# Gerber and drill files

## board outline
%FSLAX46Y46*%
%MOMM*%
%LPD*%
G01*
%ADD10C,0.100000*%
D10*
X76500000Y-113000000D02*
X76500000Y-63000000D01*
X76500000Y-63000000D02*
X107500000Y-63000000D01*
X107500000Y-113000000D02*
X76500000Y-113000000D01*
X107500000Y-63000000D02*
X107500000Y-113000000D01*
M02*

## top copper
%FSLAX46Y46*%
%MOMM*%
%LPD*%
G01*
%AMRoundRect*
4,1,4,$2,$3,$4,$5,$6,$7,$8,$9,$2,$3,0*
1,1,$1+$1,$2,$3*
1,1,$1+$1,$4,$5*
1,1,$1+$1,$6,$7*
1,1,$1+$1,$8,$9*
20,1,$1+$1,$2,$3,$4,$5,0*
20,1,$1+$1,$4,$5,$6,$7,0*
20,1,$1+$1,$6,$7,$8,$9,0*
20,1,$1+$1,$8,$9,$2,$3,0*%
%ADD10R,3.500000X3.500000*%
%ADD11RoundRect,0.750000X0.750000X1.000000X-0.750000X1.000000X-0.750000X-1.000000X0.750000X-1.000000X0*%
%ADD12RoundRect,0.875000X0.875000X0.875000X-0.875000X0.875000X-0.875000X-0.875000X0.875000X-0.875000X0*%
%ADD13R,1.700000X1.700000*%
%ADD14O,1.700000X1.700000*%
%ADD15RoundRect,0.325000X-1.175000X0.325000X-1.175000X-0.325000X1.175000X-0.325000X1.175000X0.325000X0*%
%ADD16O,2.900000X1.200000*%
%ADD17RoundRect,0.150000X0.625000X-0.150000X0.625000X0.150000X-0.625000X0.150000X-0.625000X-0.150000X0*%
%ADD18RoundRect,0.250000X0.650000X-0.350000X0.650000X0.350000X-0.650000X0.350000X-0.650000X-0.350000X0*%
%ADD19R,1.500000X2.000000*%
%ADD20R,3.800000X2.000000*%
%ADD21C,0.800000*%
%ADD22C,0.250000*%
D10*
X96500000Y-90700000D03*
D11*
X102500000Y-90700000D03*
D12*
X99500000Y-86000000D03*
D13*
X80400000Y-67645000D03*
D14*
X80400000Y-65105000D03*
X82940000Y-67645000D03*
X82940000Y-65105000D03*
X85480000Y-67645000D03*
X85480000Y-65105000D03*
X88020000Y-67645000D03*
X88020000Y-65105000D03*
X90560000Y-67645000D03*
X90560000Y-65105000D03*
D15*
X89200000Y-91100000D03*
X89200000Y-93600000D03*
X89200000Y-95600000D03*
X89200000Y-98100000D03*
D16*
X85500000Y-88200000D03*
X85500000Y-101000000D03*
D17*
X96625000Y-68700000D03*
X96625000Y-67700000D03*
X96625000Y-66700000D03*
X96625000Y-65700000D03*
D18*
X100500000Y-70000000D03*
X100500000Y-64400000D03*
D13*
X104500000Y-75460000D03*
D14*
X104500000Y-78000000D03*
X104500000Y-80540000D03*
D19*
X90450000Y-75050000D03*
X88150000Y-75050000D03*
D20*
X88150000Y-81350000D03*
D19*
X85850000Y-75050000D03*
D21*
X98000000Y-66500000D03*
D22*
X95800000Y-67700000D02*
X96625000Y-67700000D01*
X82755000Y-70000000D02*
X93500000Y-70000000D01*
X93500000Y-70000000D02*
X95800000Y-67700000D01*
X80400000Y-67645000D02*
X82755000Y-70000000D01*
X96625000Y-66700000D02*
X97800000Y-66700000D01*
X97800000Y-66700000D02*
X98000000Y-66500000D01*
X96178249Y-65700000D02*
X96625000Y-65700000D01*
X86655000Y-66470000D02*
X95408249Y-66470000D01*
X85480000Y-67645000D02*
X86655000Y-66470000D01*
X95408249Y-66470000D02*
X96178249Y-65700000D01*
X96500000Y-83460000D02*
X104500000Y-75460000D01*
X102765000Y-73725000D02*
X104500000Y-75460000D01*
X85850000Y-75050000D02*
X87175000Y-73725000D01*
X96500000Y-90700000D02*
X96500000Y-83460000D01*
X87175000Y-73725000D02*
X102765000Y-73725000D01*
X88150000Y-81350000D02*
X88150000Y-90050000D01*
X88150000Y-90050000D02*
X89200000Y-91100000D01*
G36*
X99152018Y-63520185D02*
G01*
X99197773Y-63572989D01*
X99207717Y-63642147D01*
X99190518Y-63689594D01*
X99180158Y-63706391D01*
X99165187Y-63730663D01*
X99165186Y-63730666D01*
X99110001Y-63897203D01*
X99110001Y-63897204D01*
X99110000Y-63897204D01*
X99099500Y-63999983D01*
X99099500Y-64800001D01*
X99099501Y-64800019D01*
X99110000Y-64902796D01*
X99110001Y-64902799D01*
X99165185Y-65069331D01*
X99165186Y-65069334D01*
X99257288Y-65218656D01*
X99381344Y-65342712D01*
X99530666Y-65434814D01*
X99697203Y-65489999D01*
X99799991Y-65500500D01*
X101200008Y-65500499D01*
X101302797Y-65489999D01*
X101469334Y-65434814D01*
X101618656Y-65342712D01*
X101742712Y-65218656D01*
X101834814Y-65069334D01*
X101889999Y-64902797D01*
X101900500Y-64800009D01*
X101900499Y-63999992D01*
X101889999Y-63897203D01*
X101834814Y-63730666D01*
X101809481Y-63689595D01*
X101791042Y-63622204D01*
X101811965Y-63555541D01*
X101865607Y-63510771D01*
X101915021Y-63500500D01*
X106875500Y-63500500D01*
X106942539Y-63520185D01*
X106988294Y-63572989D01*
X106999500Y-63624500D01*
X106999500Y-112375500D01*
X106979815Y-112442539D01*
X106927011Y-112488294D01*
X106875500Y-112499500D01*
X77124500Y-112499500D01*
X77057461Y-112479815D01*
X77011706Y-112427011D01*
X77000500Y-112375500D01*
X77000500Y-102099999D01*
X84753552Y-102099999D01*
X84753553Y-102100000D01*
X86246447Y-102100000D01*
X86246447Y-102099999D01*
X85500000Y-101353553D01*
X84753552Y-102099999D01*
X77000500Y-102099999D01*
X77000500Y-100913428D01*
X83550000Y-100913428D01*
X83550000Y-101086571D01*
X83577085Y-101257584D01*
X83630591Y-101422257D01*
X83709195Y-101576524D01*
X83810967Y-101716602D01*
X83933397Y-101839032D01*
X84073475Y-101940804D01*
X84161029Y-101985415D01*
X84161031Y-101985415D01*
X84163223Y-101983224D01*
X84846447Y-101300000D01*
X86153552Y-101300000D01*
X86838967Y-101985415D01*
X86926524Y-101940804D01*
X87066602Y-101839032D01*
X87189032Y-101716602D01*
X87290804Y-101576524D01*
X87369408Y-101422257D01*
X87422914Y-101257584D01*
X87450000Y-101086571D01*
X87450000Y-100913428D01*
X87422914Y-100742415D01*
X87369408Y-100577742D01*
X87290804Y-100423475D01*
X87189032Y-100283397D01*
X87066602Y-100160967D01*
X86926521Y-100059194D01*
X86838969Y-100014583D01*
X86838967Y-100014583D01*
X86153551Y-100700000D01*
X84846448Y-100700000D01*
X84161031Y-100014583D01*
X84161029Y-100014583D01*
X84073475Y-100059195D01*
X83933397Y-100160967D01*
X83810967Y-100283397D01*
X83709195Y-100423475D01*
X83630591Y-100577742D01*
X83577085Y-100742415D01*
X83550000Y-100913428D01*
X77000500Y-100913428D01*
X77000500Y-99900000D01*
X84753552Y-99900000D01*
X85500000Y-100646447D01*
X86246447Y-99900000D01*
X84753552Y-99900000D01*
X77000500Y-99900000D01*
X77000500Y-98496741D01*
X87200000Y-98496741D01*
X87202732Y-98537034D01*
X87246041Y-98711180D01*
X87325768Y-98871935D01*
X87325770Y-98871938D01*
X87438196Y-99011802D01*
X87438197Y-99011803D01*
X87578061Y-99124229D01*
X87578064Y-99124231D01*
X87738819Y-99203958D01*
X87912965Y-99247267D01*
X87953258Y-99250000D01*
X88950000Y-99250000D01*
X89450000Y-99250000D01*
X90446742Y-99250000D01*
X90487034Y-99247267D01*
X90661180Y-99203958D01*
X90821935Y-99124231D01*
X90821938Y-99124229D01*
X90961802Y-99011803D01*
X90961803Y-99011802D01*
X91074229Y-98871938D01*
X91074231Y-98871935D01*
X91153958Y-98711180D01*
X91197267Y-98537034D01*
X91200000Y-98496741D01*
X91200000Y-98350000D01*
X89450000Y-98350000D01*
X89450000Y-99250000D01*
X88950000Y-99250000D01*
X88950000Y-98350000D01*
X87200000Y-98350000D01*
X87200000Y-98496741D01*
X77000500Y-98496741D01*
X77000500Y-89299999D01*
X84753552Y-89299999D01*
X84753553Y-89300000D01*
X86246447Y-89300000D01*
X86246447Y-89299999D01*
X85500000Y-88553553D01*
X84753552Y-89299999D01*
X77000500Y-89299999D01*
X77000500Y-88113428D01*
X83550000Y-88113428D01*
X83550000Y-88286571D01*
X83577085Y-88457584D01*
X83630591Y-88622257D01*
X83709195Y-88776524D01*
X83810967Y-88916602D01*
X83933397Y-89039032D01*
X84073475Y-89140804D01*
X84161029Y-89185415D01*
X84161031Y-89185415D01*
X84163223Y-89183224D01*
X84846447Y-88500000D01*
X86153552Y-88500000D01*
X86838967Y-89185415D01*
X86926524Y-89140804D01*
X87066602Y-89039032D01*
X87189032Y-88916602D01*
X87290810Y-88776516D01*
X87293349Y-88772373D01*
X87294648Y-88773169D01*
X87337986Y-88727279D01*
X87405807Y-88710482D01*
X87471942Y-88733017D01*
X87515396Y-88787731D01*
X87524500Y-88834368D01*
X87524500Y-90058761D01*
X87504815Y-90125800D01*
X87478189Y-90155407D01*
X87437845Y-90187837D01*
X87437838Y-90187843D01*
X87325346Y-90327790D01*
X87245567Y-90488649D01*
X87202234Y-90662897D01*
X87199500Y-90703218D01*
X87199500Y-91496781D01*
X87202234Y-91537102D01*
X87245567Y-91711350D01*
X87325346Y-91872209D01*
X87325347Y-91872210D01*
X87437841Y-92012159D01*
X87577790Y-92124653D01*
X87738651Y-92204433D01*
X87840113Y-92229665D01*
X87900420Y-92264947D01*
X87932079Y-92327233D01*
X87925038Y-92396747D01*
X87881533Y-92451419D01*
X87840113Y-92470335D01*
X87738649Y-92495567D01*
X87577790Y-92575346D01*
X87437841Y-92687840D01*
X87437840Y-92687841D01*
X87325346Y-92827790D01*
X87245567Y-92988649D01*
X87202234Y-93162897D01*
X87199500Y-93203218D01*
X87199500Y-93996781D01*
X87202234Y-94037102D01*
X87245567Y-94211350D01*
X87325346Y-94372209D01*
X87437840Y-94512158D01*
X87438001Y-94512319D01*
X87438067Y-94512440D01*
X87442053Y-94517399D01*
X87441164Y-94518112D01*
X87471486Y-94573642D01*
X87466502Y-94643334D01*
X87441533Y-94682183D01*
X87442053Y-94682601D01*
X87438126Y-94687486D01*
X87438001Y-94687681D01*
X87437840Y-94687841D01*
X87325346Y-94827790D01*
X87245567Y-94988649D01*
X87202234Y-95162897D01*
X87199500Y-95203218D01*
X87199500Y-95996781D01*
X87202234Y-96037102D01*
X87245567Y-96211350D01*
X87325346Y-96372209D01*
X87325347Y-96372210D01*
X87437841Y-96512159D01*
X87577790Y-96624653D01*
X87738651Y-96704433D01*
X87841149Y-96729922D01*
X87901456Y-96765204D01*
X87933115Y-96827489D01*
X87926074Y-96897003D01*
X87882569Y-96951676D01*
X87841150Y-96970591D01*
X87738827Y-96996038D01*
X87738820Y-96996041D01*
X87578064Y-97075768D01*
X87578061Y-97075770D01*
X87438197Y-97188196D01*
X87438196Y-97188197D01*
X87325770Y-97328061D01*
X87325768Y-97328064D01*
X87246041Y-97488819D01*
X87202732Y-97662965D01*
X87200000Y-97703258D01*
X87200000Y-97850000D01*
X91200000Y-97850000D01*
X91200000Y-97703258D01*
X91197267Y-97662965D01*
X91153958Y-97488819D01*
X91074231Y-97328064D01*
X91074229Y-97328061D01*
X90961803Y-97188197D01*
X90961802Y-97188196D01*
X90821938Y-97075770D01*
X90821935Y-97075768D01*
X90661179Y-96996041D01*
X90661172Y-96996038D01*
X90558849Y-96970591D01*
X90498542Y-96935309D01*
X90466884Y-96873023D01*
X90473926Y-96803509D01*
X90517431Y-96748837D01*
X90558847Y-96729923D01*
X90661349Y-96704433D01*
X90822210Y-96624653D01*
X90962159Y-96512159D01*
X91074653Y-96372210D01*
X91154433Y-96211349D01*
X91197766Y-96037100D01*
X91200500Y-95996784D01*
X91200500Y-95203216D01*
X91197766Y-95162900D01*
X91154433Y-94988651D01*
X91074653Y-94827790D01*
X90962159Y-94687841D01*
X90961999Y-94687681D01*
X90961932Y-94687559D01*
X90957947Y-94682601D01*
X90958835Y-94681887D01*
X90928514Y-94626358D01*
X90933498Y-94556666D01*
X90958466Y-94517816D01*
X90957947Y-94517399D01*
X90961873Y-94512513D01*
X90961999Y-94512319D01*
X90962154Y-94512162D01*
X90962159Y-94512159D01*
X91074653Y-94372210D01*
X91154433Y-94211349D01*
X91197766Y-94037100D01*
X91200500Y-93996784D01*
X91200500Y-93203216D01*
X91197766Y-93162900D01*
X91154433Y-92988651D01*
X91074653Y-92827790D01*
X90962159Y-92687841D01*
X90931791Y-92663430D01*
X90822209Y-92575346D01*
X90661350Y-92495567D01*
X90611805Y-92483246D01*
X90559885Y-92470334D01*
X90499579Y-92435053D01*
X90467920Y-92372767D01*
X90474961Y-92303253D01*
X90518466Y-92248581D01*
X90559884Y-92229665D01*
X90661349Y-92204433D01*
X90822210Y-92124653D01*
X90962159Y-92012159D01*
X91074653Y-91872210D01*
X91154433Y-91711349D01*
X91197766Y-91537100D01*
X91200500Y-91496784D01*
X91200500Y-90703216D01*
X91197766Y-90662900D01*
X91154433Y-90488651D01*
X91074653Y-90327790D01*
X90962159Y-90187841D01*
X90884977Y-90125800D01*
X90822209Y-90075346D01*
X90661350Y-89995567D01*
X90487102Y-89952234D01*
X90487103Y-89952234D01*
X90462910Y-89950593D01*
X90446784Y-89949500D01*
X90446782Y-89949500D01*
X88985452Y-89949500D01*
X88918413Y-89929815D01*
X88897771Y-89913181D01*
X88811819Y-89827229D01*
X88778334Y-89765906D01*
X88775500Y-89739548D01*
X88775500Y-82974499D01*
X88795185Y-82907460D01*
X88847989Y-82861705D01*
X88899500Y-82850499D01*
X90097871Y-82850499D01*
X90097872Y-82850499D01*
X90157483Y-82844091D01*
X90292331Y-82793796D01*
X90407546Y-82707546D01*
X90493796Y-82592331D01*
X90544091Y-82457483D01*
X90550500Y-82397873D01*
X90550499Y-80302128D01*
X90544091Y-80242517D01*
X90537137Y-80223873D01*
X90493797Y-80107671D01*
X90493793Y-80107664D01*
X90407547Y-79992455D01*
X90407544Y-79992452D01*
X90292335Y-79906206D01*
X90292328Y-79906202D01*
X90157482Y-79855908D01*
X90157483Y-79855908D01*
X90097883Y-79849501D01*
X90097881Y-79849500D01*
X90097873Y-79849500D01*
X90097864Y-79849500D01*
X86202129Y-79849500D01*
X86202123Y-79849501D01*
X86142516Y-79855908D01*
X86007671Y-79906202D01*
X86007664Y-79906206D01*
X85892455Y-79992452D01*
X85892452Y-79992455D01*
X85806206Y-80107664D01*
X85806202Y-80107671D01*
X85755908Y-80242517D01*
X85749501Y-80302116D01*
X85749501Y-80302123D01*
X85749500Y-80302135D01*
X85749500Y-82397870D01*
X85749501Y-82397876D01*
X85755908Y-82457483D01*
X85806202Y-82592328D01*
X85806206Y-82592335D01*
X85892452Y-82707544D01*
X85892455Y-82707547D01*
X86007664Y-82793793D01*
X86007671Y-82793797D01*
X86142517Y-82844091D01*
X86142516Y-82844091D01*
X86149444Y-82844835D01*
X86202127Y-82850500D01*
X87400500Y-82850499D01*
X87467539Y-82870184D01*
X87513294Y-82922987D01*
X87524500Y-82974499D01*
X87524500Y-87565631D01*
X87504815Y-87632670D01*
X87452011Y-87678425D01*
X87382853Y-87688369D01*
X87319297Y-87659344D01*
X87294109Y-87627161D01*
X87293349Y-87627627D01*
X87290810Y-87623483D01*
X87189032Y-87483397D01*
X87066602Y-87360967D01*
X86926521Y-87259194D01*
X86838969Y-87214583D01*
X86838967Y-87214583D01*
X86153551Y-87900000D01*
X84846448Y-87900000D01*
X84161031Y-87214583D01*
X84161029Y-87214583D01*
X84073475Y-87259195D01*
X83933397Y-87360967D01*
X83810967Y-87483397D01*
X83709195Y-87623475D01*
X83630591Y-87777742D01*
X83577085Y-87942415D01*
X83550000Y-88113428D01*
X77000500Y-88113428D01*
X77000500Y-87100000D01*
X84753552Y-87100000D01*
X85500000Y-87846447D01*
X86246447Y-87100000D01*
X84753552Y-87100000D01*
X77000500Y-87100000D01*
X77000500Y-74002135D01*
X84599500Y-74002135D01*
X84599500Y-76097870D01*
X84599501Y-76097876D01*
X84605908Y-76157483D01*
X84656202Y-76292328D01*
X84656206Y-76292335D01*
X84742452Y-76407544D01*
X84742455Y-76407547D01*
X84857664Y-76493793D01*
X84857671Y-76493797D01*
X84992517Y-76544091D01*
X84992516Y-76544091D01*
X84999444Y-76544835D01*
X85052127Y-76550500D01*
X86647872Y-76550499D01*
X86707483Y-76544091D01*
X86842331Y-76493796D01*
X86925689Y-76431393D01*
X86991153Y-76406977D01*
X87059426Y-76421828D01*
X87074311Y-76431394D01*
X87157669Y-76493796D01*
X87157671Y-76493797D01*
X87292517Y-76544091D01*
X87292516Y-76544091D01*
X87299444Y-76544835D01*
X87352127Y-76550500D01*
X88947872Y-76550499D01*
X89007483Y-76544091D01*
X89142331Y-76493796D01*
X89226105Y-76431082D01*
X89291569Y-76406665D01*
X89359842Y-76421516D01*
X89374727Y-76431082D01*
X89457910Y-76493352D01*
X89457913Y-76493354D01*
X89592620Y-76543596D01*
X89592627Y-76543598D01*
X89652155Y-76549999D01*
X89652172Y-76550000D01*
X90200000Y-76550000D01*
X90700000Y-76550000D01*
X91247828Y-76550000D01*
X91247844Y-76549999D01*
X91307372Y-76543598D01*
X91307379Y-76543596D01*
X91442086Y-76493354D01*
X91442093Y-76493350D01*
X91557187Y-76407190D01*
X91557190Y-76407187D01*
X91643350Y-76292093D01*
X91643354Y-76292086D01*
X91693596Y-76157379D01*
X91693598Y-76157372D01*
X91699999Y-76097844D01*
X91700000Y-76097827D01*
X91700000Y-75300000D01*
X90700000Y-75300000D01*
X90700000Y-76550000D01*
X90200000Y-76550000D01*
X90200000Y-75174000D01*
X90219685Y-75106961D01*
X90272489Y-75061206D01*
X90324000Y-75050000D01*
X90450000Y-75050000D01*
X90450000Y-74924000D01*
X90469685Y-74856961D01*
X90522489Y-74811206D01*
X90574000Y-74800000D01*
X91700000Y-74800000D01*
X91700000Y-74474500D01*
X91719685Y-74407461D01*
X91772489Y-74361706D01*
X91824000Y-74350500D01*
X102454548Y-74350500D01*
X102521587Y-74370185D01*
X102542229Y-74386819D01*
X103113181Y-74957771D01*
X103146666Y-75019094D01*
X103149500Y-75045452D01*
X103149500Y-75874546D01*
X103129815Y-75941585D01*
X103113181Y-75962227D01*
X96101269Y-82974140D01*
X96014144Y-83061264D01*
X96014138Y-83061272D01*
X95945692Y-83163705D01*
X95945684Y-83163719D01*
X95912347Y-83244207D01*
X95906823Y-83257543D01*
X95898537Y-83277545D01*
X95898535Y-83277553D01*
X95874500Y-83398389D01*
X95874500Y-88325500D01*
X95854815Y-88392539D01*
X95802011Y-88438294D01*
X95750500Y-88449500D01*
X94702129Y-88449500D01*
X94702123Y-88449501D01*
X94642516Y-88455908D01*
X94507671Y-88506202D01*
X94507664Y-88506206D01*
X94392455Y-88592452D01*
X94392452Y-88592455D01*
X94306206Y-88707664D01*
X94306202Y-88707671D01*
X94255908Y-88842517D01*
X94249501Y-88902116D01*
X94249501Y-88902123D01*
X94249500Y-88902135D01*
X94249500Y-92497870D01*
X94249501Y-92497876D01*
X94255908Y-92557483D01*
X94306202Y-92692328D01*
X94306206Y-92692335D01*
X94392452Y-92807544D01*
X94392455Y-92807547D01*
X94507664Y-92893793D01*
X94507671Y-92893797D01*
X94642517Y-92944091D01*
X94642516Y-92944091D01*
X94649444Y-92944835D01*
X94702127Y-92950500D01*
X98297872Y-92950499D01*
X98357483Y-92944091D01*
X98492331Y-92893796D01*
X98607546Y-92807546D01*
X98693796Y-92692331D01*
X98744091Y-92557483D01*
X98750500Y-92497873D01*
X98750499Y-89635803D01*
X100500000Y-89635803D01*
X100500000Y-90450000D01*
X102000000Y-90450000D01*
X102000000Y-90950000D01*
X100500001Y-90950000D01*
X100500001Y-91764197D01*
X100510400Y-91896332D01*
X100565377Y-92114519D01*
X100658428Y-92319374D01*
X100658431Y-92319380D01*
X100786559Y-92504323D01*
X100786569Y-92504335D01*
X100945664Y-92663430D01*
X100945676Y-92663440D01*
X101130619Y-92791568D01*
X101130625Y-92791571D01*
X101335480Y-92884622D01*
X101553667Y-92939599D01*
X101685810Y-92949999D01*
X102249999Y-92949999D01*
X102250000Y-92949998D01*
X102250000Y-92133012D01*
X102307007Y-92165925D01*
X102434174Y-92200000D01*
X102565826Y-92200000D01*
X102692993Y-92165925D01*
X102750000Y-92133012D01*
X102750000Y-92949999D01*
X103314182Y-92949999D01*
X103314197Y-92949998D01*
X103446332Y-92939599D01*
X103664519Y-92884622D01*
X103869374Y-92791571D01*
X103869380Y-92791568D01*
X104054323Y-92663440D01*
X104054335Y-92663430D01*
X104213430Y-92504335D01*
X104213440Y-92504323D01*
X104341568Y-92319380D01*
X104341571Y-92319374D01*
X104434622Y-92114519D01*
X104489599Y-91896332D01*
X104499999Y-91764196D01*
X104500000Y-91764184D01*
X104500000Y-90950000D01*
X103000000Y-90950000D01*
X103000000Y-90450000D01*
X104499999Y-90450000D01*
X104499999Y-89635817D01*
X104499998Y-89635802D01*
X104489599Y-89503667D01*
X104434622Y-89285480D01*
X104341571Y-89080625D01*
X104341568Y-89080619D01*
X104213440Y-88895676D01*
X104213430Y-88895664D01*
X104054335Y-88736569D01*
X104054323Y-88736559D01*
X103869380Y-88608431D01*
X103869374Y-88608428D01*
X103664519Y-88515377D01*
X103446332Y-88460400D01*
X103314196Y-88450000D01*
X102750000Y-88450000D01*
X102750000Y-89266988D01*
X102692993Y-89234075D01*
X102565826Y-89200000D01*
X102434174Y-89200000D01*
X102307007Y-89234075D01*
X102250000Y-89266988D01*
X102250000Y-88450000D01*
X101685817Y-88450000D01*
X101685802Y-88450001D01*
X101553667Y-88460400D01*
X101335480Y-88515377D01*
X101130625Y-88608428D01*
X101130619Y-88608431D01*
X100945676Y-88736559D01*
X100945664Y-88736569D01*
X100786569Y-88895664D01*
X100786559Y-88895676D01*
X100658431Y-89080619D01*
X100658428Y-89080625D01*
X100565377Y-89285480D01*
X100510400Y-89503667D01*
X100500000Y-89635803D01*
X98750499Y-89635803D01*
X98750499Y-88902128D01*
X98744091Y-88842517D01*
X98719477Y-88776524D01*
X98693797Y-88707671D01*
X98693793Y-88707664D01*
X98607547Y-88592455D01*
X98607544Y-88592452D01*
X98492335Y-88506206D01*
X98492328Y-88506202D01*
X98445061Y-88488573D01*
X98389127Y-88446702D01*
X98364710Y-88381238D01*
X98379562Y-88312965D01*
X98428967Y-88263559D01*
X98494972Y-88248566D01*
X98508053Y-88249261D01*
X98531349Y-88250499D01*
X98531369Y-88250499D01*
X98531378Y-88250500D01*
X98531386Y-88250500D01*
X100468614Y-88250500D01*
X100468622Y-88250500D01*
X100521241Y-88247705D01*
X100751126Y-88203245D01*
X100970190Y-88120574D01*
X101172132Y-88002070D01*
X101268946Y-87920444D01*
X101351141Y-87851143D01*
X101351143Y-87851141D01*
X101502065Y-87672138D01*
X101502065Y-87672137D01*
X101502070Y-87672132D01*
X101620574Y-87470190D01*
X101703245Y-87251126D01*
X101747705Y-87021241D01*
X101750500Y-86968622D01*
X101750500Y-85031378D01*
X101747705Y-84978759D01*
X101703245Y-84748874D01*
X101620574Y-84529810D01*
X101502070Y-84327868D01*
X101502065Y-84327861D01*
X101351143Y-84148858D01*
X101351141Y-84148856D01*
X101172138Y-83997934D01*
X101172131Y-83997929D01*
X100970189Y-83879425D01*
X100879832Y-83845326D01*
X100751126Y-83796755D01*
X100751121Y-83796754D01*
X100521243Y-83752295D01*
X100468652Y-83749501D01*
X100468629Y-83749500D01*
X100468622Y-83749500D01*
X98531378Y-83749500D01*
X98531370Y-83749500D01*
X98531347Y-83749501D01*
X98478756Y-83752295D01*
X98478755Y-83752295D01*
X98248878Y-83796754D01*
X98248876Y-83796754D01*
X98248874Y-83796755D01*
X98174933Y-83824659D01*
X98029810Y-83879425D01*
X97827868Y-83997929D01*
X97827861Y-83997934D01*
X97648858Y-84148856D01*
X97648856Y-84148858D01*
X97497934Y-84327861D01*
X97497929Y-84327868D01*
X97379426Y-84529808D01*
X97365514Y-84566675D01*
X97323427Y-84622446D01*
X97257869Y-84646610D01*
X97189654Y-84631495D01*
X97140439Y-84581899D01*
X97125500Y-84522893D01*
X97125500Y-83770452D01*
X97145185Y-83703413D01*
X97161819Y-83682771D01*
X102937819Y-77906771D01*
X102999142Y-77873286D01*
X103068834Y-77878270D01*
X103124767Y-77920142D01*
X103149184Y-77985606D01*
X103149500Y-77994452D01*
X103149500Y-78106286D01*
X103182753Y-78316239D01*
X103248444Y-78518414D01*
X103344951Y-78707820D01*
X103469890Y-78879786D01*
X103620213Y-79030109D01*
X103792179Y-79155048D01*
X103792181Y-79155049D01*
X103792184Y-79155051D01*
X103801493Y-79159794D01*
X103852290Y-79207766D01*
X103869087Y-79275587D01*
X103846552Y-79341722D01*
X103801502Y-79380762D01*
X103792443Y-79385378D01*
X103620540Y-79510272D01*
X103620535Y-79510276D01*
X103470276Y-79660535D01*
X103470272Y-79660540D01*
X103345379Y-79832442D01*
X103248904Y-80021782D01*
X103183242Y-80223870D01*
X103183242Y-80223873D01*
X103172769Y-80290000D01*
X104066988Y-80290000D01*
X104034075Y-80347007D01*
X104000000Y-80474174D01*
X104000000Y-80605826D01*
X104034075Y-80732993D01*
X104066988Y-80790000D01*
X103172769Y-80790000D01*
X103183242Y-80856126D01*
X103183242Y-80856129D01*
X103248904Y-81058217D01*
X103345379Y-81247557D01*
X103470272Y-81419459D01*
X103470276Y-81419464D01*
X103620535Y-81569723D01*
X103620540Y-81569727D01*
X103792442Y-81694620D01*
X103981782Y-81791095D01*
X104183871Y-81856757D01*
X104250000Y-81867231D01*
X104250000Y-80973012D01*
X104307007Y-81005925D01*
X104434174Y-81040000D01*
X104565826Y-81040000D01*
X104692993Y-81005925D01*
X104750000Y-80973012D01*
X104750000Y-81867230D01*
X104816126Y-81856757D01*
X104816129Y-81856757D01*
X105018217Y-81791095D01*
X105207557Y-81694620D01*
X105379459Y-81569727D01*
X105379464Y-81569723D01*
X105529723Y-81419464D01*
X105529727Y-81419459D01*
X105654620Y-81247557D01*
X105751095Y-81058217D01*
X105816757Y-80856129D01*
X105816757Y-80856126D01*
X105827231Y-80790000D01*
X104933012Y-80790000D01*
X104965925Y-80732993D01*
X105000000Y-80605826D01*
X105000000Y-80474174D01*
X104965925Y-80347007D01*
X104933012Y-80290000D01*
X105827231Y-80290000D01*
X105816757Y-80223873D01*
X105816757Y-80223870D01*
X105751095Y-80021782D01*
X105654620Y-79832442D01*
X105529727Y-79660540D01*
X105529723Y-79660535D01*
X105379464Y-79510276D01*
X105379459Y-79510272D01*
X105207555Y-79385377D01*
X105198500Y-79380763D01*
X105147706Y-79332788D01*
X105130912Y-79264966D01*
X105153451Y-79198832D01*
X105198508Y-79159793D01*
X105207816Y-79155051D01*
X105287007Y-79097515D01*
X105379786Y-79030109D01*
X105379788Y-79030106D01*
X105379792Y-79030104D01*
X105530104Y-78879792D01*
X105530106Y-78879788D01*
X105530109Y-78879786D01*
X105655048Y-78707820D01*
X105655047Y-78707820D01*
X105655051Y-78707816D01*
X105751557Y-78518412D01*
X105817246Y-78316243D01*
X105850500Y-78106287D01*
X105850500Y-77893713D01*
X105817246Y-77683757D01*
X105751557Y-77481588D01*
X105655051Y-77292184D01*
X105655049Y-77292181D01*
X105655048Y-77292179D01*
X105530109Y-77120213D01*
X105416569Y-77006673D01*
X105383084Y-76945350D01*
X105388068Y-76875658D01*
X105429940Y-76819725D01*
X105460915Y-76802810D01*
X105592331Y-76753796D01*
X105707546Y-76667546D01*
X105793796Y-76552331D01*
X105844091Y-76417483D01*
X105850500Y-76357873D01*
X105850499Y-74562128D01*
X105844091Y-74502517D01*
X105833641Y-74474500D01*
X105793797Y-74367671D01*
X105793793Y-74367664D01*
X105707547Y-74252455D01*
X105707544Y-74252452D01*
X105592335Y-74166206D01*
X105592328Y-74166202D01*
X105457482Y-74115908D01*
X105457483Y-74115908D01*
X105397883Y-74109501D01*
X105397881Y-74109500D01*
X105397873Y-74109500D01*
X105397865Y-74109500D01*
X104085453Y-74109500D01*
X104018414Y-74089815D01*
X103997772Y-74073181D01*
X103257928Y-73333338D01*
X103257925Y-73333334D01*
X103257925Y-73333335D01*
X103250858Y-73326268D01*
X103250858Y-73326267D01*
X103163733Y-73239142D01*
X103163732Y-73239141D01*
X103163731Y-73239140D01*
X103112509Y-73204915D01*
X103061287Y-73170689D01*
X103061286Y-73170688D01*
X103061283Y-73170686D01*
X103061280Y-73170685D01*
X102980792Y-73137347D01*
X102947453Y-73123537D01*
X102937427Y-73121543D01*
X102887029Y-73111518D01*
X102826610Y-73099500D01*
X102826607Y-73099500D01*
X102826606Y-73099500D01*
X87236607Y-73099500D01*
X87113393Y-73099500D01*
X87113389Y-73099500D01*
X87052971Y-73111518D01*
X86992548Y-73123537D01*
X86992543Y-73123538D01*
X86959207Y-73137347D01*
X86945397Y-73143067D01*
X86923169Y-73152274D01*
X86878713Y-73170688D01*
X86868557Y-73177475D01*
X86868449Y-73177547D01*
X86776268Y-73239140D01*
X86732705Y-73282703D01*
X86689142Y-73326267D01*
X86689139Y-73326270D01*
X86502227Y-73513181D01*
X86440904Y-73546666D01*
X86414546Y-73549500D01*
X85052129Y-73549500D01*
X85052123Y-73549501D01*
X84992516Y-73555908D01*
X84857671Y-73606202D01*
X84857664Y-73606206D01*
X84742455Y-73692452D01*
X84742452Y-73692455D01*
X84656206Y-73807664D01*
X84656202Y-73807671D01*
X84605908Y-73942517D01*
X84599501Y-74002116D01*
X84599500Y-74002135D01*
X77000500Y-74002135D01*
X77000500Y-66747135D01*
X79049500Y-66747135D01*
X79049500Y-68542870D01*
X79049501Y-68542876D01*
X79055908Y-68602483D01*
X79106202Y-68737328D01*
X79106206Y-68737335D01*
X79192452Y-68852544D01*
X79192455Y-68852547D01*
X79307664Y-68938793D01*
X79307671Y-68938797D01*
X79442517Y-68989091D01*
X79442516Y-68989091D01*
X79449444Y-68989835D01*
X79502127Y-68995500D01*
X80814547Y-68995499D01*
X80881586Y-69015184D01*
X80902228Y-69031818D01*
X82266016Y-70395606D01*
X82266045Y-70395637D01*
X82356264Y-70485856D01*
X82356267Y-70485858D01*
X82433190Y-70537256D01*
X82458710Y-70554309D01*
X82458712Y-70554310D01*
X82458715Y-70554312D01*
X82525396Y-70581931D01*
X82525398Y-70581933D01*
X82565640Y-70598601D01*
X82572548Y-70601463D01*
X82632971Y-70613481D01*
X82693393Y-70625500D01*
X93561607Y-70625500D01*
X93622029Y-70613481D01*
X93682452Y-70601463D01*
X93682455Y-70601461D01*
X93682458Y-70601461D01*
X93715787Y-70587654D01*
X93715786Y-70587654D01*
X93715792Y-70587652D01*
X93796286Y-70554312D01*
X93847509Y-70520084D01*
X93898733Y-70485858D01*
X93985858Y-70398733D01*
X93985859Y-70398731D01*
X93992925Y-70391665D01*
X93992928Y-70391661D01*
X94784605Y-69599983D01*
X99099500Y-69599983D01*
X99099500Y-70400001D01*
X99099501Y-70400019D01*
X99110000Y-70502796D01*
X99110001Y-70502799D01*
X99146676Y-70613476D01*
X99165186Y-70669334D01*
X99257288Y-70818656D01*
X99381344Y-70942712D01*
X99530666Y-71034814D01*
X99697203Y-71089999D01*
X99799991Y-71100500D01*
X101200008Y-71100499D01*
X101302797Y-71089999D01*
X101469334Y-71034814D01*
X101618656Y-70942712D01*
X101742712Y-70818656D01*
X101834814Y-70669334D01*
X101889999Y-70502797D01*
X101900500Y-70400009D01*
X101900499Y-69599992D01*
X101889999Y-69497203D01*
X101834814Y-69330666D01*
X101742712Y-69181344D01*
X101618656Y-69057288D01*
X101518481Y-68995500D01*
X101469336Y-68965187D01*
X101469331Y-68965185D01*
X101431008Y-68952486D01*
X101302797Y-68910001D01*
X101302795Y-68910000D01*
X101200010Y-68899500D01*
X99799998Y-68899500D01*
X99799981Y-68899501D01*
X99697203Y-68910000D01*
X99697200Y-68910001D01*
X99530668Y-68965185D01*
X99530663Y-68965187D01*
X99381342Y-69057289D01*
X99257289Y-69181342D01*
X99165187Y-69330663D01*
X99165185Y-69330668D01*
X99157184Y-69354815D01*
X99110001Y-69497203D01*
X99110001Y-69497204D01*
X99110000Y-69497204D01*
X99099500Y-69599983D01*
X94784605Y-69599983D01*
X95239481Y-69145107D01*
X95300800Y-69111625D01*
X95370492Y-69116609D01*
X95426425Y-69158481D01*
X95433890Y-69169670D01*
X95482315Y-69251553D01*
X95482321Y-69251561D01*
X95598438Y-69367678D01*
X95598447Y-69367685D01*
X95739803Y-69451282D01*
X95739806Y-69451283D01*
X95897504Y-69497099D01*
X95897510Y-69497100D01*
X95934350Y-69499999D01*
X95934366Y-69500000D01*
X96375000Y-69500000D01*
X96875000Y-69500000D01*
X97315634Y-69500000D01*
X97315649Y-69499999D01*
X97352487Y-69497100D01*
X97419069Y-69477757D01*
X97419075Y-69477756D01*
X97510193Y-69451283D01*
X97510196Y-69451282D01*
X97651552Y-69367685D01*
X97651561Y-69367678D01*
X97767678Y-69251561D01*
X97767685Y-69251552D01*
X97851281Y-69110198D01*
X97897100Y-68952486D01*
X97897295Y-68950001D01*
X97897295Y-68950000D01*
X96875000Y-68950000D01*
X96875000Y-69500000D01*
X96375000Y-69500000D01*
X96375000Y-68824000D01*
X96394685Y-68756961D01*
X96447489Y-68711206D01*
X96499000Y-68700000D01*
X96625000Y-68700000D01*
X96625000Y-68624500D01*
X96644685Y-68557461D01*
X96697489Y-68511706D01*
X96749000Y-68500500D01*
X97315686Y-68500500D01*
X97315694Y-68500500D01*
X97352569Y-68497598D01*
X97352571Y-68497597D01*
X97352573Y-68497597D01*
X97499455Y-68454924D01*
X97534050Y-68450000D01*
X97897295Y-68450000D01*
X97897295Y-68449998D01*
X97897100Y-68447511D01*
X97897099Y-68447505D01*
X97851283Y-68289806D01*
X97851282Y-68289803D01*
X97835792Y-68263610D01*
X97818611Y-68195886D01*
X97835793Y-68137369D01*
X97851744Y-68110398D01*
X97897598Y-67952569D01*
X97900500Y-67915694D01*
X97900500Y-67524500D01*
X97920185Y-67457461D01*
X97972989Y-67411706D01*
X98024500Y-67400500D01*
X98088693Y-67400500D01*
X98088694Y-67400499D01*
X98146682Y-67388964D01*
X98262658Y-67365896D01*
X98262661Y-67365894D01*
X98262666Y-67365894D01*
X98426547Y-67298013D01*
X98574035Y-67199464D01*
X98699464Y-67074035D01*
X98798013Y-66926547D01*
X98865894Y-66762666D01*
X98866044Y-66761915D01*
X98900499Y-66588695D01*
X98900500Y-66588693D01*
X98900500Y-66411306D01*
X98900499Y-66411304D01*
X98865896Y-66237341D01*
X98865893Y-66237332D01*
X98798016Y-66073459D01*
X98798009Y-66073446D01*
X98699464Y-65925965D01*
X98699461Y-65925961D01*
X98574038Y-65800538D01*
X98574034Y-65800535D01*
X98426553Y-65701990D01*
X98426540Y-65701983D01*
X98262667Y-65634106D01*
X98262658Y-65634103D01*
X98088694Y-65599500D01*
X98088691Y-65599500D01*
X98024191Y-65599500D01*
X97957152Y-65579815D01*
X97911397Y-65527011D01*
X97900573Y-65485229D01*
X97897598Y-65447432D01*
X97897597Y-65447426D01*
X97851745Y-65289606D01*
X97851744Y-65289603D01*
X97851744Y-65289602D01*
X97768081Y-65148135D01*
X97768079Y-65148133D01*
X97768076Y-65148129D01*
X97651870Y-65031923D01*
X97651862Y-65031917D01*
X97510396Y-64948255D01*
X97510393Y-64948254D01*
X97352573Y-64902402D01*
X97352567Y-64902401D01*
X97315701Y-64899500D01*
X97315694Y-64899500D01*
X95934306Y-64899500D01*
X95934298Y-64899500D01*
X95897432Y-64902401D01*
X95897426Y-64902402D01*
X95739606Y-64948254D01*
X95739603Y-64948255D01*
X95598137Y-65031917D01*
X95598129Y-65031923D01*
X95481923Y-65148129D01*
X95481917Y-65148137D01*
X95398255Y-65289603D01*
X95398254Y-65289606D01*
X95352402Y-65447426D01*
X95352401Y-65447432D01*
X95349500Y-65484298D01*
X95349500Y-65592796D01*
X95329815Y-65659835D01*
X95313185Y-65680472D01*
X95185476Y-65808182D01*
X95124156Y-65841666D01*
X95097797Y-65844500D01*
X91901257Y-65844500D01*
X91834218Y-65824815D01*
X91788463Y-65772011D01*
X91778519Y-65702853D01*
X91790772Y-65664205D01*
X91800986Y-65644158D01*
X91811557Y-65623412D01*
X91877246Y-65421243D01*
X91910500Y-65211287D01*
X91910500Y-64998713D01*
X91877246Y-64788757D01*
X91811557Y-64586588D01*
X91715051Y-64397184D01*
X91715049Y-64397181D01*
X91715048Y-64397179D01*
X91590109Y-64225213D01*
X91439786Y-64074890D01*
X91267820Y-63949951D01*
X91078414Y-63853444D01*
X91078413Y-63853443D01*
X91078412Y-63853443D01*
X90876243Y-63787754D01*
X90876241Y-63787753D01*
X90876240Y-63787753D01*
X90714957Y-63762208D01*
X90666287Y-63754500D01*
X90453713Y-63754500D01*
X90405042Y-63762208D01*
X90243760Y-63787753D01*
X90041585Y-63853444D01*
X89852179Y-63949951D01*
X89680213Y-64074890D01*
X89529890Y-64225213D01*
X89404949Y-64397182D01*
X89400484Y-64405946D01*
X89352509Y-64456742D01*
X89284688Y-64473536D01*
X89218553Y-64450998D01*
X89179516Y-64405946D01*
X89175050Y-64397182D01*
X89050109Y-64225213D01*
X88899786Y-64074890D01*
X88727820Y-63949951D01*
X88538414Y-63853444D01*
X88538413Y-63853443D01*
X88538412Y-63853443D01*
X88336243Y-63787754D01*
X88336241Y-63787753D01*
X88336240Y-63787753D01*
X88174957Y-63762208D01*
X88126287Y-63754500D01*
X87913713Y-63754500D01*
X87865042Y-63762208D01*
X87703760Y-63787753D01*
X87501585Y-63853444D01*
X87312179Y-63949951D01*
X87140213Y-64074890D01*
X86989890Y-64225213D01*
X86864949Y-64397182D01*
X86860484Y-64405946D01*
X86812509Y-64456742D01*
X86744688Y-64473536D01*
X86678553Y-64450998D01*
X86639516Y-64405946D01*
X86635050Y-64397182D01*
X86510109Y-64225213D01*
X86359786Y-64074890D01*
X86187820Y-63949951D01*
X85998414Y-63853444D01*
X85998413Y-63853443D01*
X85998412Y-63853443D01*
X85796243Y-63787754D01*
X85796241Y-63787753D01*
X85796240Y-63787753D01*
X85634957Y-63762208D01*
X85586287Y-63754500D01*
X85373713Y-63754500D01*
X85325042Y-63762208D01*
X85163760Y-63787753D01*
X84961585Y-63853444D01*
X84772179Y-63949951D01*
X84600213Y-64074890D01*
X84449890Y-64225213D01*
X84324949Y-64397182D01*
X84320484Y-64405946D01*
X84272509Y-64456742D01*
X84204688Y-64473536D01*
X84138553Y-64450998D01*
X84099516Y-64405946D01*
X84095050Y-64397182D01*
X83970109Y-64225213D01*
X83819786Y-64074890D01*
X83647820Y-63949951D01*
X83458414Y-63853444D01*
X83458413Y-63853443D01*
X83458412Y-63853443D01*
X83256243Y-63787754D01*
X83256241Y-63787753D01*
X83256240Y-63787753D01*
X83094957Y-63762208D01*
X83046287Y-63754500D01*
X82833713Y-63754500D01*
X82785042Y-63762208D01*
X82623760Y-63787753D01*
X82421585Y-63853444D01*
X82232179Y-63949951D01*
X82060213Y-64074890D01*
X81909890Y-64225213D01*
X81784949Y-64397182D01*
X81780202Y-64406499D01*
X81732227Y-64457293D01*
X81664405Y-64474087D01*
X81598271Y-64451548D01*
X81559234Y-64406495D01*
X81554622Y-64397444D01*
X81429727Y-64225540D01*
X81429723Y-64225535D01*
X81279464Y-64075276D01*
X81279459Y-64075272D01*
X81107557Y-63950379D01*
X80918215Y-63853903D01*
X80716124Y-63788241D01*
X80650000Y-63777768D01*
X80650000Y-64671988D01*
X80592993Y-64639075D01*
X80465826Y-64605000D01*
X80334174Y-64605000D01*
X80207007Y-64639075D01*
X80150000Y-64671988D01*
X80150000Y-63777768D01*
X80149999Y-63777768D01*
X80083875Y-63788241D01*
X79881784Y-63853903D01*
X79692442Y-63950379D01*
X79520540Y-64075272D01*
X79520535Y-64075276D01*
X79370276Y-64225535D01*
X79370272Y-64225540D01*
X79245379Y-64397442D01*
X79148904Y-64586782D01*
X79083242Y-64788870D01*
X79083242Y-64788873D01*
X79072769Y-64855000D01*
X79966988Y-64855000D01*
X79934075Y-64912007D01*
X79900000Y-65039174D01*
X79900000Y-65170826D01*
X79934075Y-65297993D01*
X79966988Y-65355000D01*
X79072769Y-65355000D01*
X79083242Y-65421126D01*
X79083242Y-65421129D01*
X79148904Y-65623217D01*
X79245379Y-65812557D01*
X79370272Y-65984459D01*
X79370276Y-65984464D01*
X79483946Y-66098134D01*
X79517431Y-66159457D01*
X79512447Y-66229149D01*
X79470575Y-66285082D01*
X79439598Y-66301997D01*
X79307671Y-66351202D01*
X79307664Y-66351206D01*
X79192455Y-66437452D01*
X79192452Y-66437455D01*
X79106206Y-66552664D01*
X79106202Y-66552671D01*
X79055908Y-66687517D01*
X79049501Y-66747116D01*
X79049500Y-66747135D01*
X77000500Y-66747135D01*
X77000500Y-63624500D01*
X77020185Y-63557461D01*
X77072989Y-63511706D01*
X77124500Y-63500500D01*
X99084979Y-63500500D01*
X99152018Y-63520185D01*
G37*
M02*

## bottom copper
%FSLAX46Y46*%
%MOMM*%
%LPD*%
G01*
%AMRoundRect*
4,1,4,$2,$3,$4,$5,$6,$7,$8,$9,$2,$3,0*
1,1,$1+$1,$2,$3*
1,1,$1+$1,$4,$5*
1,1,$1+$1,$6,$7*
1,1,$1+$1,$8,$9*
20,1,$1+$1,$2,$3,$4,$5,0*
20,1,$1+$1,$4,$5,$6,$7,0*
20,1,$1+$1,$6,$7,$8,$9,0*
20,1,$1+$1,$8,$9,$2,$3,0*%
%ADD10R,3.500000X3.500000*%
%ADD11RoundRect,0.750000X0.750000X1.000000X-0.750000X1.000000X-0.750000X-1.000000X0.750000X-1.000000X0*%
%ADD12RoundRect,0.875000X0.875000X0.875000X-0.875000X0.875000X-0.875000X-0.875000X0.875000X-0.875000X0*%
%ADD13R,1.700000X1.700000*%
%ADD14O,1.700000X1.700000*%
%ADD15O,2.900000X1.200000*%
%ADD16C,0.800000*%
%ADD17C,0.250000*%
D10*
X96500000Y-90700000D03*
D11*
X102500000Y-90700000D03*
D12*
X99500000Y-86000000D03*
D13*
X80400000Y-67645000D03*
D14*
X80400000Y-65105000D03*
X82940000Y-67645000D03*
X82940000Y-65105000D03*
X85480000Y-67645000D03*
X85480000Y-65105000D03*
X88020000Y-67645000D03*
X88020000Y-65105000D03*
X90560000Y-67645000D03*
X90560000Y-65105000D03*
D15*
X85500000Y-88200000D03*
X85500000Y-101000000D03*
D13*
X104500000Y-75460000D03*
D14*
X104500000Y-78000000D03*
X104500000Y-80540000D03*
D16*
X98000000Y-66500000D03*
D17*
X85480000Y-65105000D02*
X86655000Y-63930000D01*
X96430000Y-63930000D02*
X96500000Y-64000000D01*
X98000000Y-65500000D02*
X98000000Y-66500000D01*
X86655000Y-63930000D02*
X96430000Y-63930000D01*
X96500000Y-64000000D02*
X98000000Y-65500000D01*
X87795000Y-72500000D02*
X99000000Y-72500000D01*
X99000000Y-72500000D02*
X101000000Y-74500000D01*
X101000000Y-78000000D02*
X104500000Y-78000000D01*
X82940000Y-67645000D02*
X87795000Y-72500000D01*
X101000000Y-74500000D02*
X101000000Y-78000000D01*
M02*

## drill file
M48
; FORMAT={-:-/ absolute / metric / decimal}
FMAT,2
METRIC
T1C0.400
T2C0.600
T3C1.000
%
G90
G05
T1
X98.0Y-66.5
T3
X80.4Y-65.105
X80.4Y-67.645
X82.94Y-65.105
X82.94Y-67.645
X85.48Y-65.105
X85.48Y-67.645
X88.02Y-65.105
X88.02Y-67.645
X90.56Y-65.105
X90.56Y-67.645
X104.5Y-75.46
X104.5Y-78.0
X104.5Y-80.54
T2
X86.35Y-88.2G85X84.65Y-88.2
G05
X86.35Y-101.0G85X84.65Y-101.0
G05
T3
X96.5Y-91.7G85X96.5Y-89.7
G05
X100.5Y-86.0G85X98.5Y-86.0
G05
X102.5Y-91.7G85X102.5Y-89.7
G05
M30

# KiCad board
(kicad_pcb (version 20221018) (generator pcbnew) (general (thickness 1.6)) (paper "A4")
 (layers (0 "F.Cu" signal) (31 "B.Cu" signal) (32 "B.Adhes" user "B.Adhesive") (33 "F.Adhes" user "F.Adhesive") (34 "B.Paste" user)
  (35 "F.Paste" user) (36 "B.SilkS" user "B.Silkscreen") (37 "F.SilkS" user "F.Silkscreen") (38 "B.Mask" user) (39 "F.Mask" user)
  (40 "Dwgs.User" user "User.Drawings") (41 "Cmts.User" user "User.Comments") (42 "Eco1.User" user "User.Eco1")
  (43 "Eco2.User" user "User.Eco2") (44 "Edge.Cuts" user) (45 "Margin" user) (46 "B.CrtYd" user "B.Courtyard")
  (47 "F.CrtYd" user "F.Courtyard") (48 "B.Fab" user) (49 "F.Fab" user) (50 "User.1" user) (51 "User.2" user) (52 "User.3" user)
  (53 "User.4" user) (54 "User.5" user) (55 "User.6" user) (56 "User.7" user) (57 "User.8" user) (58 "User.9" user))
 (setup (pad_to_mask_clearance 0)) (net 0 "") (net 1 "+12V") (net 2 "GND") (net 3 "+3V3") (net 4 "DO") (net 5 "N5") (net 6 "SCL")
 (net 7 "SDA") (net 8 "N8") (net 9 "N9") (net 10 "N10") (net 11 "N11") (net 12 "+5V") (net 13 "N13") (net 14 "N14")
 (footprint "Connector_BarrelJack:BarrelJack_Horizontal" (layer "F.Cu") (at 96.5 90.7 180)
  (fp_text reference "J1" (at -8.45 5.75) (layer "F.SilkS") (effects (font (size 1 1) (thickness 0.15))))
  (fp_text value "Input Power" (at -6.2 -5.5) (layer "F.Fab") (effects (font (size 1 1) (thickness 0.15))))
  (pad "1" thru_hole rect (at 0 0 180) (size 3.5 3.5) (drill oval 1 3) (layers "*.Cu" "*.Mask") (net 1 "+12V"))
  (pad "2" thru_hole roundrect (at -6 0 180) (size 3 3.5) (drill oval 1 3) (layers "*.Cu" "*.Mask") (roundrect_rratio 0.25) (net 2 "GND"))
  (pad "3" thru_hole roundrect (at -3 4.7 180) (size 3.5 3.5) (drill oval 3 1) (layers "*.Cu" "*.Mask") (roundrect_rratio 0.25)))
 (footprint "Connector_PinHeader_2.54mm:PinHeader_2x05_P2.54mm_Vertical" (layer "F.Cu") (at 80.4 67.645 90)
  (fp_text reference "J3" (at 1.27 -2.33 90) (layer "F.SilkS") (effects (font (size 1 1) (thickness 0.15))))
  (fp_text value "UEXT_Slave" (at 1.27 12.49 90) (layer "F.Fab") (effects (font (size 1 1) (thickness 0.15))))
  (pad "1" thru_hole rect (at 0 0 90) (size 1.7 1.7) (drill 1) (layers "*.Cu" "*.Mask") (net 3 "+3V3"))
  (pad "2" thru_hole oval (at 2.54 0 90) (size 1.7 1.7) (drill 1) (layers "*.Cu" "*.Mask") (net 2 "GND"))
  (pad "3" thru_hole oval (at 0 2.54 90) (size 1.7 1.7) (drill 1) (layers "*.Cu" "*.Mask") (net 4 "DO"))
  (pad "4" thru_hole oval (at 2.54 2.54 90) (size 1.7 1.7) (drill 1) (layers "*.Cu" "*.Mask") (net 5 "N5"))
  (pad "5" thru_hole oval (at 0 5.08 90) (size 1.7 1.7) (drill 1) (layers "*.Cu" "*.Mask") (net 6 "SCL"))
  (pad "6" thru_hole oval (at 2.54 5.08 90) (size 1.7 1.7) (drill 1) (layers "*.Cu" "*.Mask") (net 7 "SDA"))
  (pad "7" thru_hole oval (at 0 7.62 90) (size 1.7 1.7) (drill 1) (layers "*.Cu" "*.Mask") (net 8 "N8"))
  (pad "8" thru_hole oval (at 2.54 7.62 90) (size 1.7 1.7) (drill 1) (layers "*.Cu" "*.Mask") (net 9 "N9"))
  (pad "9" thru_hole oval (at 0 10.16 90) (size 1.7 1.7) (drill 1) (layers "*.Cu" "*.Mask") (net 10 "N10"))
  (pad "10" thru_hole oval (at 2.54 10.16 90) (size 1.7 1.7) (drill 1) (layers "*.Cu" "*.Mask") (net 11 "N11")))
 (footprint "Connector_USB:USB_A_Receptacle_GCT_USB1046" (layer "F.Cu") (at 81.95 94.6 -90)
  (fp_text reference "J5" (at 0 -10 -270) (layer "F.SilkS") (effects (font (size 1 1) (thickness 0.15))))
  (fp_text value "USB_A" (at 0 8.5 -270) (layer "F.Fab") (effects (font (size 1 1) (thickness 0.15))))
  (pad "" smd oval (at -6.4 -3.55 270) (size 1.2 2.9) (layers "F.Paste") (thermal_bridge_angle 45))
  (pad "" smd oval (at 6.4 -3.55 270) (size 1.2 2.9) (layers "F.Paste") (thermal_bridge_angle 45))
  (pad "1" smd roundrect (at -3.5 -7.25 270) (size 1.3 3) (layers "F.Cu" "F.Paste" "F.Mask") (roundrect_rratio 0.25) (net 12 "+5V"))
  (pad "2" smd roundrect (at -1 -7.25 270) (size 1.3 3) (layers "F.Cu" "F.Paste" "F.Mask") (roundrect_rratio 0.25) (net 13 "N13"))
  (pad "3" smd roundrect (at 1 -7.25 270) (size 1.3 3) (layers "F.Cu" "F.Paste" "F.Mask") (roundrect_rratio 0.25) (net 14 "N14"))
  (pad "4" smd roundrect (at 3.5 -7.25 270) (size 1.3 3) (layers "F.Cu" "F.Paste" "F.Mask") (roundrect_rratio 0.25) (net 2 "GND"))
  (pad "5" thru_hole oval (at -6.4 -3.55 270) (size 1.2 2.9) (drill oval 0.6 2.3) (layers "*.Cu" "*.Mask") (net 2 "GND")
   (thermal_bridge_angle 45))
  (pad "5" thru_hole oval (at 6.4 -3.55 270) (size 1.2 2.9) (drill oval 0.6 2.3) (layers "*.Cu" "*.Mask") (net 2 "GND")
   (thermal_bridge_angle 45)))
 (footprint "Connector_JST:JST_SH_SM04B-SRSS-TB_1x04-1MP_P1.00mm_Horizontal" (layer "F.Cu") (at 98.625 67.2 90)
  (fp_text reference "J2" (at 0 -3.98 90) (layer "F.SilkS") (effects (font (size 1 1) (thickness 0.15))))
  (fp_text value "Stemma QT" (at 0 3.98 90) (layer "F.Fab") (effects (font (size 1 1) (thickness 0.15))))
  (pad "1" smd roundrect (at -1.5 -2 90) (size 0.6 1.55) (layers "F.Cu" "F.Paste" "F.Mask") (roundrect_rratio 0.25) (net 2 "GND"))
  (pad "2" smd roundrect (at -0.5 -2 90) (size 0.6 1.55) (layers "F.Cu" "F.Paste" "F.Mask") (roundrect_rratio 0.25) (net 3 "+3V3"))
  (pad "3" smd roundrect (at 0.5 -2 90) (size 0.6 1.55) (layers "F.Cu" "F.Paste" "F.Mask") (roundrect_rratio 0.25) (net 7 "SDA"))
  (pad "4" smd roundrect (at 1.5 -2 90) (size 0.6 1.55) (layers "F.Cu" "F.Paste" "F.Mask") (roundrect_rratio 0.25) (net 6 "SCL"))
  (pad "MP" smd roundrect (at -2.8 1.875 90) (size 1.2 1.8) (layers "F.Cu" "F.Paste" "F.Mask") (roundrect_rratio 0.208333))
  (pad "MP" smd roundrect (at 2.8 1.875 90) (size 1.2 1.8) (layers "F.Cu" "F.Paste" "F.Mask") (roundrect_rratio 0.208333)))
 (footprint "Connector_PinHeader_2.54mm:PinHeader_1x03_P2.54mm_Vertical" (layer "F.Cu") (at 104.5 75.46)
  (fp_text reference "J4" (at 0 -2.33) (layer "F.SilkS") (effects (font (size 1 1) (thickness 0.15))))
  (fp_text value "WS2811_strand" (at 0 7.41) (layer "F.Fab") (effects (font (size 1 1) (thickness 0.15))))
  (pad "1" thru_hole rect (at 0 0) (size 1.7 1.7) (drill 1) (layers "*.Cu" "*.Mask") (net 1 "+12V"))
  (pad "2" thru_hole oval (at 0 2.54) (size 1.7 1.7) (drill 1) (layers "*.Cu" "*.Mask") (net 4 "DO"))
  (pad "3" thru_hole oval (at 0 5.08) (size 1.7 1.7) (drill 1) (layers "*.Cu" "*.Mask") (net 2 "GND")))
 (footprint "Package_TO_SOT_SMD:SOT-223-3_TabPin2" (layer "F.Cu") (at 88.15 78.2 -90)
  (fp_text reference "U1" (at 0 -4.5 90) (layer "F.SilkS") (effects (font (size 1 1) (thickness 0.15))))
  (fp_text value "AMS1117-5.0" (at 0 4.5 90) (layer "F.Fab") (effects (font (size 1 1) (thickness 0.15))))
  (pad "1" smd rect (at -3.15 -2.3 270) (size 2 1.5) (layers "F.Cu" "F.Paste" "F.Mask") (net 2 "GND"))
  (pad "2" smd rect (at -3.15 0 270) (size 2 1.5) (layers "F.Cu" "F.Paste" "F.Mask") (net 12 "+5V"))
  (pad "2" smd rect (at 3.15 0 270) (size 2 3.8) (layers "F.Cu" "F.Paste" "F.Mask") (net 12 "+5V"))
  (pad "3" smd rect (at -3.15 2.3 270) (size 2 1.5) (layers "F.Cu" "F.Paste" "F.Mask") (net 1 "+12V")))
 (gr_line (start 76.5 113) (end 76.5 63) (stroke (width 0.1) (type default)) (layer "Edge.Cuts"))
 (gr_line (start 76.5 63) (end 107.5 63) (stroke (width 0.1) (type default)) (layer "Edge.Cuts"))
 (gr_line (start 107.5 113) (end 76.5 113) (stroke (width 0.1) (type default)) (layer "Edge.Cuts"))
 (gr_line (start 107.5 63) (end 107.5 113) (stroke (width 0.1) (type default)) (layer "Edge.Cuts"))
 (segment (start 95.8 67.7) (end 96.625 67.7) (width 0.25) (layer "F.Cu") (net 3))
 (segment (start 82.755 70) (end 93.5 70) (width 0.25) (layer "F.Cu") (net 3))
 (segment (start 93.5 70) (end 95.8 67.7) (width 0.25) (layer "F.Cu") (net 3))
 (segment (start 80.4 67.645) (end 82.755 70) (width 0.25) (layer "F.Cu") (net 3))
 (segment (start 96.625 66.7) (end 97.8 66.7) (width 0.25) (layer "F.Cu") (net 7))
 (segment (start 97.8 66.7) (end 98 66.5) (width 0.25) (layer "F.Cu") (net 7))
 (via (at 98 66.5) (size 0.8) (drill 0.4) (layers "F.Cu" "B.Cu") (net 7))
 (segment (start 85.48 65.105) (end 86.655 63.93) (width 0.25) (layer "B.Cu") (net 7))
 (segment (start 96.43 63.93) (end 96.5 64) (width 0.25) (layer "B.Cu") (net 7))
 (segment (start 98 65.5) (end 98 66.5) (width 0.25) (layer "B.Cu") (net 7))
 (segment (start 86.655 63.93) (end 96.43 63.93) (width 0.25) (layer "B.Cu") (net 7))
 (segment (start 96.5 64) (end 98 65.5) (width 0.25) (layer "B.Cu") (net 7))
 (segment (start 96.178249 65.7) (end 96.625 65.7) (width 0.25) (layer "F.Cu") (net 6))
 (segment (start 86.655 66.47) (end 95.408249 66.47) (width 0.25) (layer "F.Cu") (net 6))
 (segment (start 85.48 67.645) (end 86.655 66.47) (width 0.25) (layer "F.Cu") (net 6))
 (segment (start 95.408249 66.47) (end 96.178249 65.7) (width 0.25) (layer "F.Cu") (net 6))
 (segment (start 96.5 83.46) (end 104.5 75.46) (width 0.25) (layer "F.Cu") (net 1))
 (segment (start 102.765 73.725) (end 104.5 75.46) (width 0.25) (layer "F.Cu") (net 1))
 (segment (start 85.85 75.05) (end 87.175 73.725) (width 0.25) (layer "F.Cu") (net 1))
 (segment (start 96.5 90.7) (end 96.5 83.46) (width 0.25) (layer "F.Cu") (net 1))
 (segment (start 87.175 73.725) (end 102.765 73.725) (width 0.25) (layer "F.Cu") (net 1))
 (segment (start 88.15 81.35) (end 88.15 90.05) (width 0.25) (layer "F.Cu") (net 12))
 (segment (start 88.15 90.05) (end 89.2 91.1) (width 0.25) (layer "F.Cu") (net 12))
 (segment (start 87.795 72.5) (end 99 72.5) (width 0.25) (layer "B.Cu") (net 4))
 (segment (start 99 72.5) (end 101 74.5) (width 0.25) (layer "B.Cu") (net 4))
 (segment (start 101 78) (end 104.5 78) (width 0.25) (layer "B.Cu") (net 4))
 (segment (start 82.94 67.645) (end 87.795 72.5) (width 0.25) (layer "B.Cu") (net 4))
 (segment (start 101 74.5) (end 101 78) (width 0.25) (layer "B.Cu") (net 4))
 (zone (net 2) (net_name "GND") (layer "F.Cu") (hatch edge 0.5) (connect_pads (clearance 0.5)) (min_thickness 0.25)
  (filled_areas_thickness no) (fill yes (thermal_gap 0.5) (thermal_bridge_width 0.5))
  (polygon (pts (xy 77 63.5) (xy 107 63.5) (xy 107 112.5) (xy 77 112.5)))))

